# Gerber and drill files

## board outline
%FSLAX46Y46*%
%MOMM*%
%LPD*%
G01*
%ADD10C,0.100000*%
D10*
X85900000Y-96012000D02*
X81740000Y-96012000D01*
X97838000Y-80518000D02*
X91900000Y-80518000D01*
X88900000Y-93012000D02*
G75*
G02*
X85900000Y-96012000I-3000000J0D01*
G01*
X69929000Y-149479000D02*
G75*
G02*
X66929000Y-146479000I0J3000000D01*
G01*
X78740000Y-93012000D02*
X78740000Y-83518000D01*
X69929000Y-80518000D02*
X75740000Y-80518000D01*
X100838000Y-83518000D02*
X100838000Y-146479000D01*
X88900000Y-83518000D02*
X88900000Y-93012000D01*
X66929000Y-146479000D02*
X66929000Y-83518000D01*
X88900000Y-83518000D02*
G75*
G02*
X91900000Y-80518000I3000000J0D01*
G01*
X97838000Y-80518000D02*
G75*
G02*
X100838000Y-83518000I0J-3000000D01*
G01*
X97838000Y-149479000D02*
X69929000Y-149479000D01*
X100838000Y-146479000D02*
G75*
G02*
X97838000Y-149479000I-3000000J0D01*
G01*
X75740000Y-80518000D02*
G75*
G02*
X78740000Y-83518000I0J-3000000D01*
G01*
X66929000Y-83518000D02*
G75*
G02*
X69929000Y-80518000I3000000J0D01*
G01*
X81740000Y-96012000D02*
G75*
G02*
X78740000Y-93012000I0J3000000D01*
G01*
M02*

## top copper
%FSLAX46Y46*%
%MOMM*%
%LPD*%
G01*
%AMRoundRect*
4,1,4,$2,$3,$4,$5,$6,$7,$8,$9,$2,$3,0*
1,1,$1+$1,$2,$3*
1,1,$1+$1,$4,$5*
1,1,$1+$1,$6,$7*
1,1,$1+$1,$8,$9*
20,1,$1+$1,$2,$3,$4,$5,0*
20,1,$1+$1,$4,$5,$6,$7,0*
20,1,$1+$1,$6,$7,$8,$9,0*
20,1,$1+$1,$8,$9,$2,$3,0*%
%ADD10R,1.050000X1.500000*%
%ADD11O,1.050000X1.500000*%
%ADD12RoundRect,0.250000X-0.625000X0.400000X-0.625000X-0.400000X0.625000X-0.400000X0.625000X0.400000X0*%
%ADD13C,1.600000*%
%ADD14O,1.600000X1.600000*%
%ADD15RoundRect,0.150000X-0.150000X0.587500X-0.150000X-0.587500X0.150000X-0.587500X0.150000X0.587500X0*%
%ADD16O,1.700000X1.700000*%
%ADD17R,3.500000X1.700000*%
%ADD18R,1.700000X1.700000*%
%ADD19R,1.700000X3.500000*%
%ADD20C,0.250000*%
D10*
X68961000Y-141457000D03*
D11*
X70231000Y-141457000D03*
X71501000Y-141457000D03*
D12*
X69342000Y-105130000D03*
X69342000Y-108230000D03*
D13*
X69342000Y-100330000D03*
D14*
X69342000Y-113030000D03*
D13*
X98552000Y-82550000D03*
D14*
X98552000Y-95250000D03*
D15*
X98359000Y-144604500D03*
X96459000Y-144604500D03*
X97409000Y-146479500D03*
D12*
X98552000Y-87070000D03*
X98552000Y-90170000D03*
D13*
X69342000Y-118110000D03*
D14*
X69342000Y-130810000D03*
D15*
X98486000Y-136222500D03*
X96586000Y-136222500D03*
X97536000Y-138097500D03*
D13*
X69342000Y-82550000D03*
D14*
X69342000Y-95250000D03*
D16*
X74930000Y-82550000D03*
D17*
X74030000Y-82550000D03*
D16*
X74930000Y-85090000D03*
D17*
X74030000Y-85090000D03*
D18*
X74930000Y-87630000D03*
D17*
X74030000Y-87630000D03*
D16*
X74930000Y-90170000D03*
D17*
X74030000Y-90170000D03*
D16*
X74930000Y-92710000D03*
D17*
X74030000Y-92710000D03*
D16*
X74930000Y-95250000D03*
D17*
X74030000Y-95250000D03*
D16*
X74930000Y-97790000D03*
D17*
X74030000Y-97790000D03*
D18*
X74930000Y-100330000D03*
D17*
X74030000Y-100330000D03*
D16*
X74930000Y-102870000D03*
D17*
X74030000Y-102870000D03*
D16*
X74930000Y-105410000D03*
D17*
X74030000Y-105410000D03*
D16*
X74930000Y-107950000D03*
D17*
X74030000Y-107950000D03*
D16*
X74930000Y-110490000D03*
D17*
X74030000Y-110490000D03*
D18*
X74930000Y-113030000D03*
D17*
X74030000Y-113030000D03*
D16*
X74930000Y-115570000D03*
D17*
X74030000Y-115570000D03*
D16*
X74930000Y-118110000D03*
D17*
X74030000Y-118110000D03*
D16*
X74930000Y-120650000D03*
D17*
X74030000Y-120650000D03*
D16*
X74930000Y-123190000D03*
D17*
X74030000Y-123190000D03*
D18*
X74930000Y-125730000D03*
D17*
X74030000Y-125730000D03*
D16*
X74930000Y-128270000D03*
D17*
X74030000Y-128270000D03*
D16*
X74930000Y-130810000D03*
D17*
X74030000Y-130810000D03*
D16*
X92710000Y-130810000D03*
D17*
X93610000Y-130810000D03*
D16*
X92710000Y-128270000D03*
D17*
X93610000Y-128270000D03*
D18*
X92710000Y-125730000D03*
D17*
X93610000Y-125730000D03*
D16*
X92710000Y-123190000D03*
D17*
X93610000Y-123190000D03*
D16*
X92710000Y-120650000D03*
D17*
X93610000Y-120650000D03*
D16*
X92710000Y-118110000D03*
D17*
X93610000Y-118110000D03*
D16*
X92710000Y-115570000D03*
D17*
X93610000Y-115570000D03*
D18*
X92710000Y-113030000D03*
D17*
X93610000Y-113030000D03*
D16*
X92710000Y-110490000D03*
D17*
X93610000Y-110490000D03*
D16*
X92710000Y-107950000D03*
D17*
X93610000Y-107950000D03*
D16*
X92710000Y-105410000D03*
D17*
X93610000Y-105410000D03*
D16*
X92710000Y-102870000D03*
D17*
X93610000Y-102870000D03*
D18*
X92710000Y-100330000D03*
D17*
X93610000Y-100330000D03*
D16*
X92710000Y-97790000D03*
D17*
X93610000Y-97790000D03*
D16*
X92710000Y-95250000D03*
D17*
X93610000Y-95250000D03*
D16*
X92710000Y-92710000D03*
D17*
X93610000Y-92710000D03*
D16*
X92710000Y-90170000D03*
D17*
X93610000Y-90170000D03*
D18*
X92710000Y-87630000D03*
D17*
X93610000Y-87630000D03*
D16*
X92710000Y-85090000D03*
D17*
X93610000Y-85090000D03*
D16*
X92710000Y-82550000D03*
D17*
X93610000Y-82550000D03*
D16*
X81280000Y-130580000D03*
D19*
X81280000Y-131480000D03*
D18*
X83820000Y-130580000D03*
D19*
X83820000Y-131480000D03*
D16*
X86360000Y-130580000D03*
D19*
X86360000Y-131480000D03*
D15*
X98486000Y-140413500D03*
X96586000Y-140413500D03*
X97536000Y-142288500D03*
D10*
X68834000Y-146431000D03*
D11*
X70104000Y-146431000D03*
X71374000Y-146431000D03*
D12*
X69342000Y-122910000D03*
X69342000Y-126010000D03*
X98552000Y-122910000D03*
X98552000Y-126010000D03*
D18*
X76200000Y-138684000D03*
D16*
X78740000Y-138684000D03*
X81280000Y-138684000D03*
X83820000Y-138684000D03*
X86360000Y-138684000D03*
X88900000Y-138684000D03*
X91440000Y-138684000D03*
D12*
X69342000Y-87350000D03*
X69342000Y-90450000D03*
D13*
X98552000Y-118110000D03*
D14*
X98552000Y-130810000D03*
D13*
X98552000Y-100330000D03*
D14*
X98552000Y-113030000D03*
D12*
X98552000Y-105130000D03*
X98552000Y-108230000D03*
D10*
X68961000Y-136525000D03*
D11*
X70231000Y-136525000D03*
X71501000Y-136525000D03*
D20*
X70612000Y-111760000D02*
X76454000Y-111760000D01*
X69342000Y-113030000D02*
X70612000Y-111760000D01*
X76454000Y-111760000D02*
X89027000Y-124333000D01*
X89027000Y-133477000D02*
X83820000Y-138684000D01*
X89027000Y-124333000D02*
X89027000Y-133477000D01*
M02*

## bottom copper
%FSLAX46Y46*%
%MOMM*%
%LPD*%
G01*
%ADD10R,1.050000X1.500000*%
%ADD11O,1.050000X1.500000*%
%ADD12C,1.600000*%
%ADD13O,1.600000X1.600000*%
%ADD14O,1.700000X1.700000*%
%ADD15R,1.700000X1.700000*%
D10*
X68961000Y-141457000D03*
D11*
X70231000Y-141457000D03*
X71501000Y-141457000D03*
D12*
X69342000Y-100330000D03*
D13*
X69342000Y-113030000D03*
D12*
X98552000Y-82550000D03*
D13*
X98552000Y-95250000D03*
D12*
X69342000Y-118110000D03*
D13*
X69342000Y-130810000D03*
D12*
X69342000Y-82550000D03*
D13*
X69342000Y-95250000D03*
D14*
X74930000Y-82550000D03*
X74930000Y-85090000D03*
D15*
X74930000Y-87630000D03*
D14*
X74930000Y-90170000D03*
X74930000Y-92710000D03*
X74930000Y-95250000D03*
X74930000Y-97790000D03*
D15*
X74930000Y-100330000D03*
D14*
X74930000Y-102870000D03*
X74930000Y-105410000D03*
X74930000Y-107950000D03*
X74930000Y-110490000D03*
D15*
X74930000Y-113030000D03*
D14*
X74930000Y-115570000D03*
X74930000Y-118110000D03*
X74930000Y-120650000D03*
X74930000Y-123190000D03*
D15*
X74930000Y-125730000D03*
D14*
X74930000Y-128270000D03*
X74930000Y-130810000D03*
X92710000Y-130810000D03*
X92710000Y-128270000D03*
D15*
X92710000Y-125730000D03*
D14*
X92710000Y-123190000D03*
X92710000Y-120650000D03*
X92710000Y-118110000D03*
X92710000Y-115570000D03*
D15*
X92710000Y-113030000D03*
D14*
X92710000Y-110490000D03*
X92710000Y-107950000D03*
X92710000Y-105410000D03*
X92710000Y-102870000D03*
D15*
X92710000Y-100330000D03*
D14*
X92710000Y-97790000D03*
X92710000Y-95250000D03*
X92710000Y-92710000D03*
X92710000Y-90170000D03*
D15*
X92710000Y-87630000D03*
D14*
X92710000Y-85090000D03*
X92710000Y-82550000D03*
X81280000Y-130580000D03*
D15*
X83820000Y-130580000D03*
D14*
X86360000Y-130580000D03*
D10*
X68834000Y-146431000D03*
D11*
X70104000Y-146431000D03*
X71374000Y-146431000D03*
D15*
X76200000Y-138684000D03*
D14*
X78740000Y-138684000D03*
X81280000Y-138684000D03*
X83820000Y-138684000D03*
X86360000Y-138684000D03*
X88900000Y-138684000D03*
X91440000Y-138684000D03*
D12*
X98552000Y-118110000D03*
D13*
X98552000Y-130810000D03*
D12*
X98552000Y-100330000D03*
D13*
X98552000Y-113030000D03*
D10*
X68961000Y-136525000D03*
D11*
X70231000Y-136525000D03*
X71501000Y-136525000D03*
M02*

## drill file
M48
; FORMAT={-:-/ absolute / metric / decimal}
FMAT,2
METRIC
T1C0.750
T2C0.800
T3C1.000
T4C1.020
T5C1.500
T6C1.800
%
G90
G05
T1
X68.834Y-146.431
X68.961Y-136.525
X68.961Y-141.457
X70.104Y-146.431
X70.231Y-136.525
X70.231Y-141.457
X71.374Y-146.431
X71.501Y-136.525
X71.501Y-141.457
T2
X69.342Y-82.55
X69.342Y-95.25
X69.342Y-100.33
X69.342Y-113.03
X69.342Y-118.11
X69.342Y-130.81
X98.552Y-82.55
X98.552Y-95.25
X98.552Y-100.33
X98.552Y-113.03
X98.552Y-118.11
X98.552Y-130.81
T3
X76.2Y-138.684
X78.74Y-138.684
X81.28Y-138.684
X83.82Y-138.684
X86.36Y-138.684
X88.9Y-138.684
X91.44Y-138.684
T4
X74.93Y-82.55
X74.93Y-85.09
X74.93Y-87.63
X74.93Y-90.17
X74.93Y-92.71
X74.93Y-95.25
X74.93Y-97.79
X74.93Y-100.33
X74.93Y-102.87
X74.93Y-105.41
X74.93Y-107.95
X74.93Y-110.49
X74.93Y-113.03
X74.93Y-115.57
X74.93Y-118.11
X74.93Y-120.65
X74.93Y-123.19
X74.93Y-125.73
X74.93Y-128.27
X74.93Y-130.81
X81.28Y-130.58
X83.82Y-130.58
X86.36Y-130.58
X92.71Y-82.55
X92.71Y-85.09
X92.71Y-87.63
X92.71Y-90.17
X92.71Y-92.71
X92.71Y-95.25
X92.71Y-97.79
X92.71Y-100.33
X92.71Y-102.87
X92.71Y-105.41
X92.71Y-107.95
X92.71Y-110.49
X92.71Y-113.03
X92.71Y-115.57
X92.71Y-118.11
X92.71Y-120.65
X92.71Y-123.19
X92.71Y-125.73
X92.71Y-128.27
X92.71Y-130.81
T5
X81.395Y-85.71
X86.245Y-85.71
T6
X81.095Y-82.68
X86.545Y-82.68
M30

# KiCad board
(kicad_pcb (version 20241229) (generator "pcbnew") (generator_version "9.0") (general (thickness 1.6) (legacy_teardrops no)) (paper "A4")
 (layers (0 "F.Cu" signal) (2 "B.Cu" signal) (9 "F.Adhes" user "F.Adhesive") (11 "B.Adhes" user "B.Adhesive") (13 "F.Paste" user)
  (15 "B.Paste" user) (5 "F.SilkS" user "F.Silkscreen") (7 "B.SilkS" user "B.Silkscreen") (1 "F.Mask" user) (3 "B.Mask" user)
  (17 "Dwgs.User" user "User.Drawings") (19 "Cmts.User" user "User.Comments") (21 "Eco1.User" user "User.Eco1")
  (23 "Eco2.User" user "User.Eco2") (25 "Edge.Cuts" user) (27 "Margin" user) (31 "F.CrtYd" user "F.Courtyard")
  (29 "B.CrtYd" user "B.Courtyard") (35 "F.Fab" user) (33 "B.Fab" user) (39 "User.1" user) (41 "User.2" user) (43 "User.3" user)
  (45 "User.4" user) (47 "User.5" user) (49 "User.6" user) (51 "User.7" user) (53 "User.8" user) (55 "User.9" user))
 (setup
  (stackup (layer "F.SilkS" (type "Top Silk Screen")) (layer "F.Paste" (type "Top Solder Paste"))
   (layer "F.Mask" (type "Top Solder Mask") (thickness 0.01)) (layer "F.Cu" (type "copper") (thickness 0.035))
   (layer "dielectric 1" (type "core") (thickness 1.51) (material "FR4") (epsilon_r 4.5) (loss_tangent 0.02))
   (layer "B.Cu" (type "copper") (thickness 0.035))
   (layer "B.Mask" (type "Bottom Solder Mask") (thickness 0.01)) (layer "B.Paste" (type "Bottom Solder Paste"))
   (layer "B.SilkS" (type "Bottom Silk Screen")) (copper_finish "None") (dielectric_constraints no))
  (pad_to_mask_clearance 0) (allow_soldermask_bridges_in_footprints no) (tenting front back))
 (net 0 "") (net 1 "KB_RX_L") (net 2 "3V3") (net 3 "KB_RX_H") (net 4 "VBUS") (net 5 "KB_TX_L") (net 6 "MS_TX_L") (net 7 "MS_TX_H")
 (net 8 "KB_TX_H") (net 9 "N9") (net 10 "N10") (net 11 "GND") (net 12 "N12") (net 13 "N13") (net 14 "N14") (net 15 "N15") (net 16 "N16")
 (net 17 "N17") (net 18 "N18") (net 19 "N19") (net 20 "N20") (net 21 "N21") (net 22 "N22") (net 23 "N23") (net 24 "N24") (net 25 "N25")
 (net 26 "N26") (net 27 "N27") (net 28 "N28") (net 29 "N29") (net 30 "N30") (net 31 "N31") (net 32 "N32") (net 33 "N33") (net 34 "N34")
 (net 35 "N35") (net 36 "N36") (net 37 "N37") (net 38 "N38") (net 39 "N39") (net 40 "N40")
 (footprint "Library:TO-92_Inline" (layer "F.Cu") (at 68.961 141.457)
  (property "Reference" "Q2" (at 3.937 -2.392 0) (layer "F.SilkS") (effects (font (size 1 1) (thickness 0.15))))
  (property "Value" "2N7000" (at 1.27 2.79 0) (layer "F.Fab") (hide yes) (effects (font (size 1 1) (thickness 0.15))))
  (pad "1" thru_hole rect (at 0 0) (size 1.05 1.5) (drill 0.75) (layers "*.Cu" "*.Mask") (remove_unused_layers no) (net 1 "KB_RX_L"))
  (pad "2" thru_hole oval (at 1.27 0) (size 1.05 1.5) (drill 0.75) (layers "*.Cu" "*.Mask") (remove_unused_layers no) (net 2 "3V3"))
  (pad "3" thru_hole oval (at 2.54 0) (size 1.05 1.5) (drill 0.75) (layers "*.Cu" "*.Mask") (remove_unused_layers no) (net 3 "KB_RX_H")))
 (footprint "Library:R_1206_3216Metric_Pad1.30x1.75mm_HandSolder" (layer "F.Cu") (at 69.342 106.68 -90)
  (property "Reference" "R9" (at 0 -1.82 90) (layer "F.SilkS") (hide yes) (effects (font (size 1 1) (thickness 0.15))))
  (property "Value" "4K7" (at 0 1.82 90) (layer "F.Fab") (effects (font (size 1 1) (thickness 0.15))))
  (pad "1" smd roundrect (at -1.55 0 270) (size 1.3 1.75) (layers "F.Cu" "F.Mask" "F.Paste") (roundrect_rratio 0.192308) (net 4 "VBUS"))
  (pad "2" smd roundrect (at 1.55 0 270) (size 1.3 1.75) (layers "F.Cu" "F.Mask" "F.Paste") (roundrect_rratio 0.192308) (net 3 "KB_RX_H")))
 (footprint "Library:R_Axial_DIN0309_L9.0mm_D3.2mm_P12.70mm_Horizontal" (layer "F.Cu") (at 69.342 100.33 -90)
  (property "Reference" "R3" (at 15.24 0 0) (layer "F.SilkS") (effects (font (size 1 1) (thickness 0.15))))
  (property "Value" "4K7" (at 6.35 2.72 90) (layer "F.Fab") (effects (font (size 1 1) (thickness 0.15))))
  (pad "1" thru_hole circle (at 0 0 270) (size 1.6 1.6) (drill 0.8) (layers "*.Cu" "*.Mask") (remove_unused_layers no) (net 4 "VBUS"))
  (pad "2" thru_hole oval (at 12.7 0 270) (size 1.6 1.6) (drill 0.8) (layers "*.Cu" "*.Mask") (remove_unused_layers no) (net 3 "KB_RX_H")))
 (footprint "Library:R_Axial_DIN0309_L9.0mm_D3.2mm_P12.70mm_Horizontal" (layer "F.Cu") (at 98.552 82.55 -90)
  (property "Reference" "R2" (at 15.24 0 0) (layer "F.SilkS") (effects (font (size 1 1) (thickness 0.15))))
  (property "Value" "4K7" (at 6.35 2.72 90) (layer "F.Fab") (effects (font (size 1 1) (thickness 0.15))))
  (pad "1" thru_hole circle (at 0 0 270) (size 1.6 1.6) (drill 0.8) (layers "*.Cu" "*.Mask") (remove_unused_layers no) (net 2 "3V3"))
  (pad "2" thru_hole oval (at 12.7 0 270) (size 1.6 1.6) (drill 0.8) (layers "*.Cu" "*.Mask") (remove_unused_layers no) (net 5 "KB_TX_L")))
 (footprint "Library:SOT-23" (layer "F.Cu") (at 97.409 145.542 -90)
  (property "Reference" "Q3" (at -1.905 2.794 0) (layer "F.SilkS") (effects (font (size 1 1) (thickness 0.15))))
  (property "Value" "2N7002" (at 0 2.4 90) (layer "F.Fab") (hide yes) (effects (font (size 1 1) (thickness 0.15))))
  (pad "1" smd roundrect (at -0.9375 -0.95 270) (size 1.475 0.6) (layers "F.Cu" "F.Mask" "F.Paste") (roundrect_rratio 0.25) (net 2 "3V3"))
  (pad "2" smd roundrect (at -0.9375 0.95 270) (size 1.475 0.6) (layers "F.Cu" "F.Mask" "F.Paste") (roundrect_rratio 0.25) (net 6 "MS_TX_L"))
  (pad "3" smd roundrect (at 0.9375 0 270) (size 1.475 0.6) (layers "F.Cu" "F.Mask" "F.Paste") (roundrect_rratio 0.25) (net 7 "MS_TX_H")))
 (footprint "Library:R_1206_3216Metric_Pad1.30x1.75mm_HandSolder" (layer "F.Cu") (at 98.552 88.62 -90)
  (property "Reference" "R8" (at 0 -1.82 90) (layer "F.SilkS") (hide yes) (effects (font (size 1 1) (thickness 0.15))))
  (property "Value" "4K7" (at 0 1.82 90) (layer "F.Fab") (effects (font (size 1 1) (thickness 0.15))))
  (pad "1" smd roundrect (at -1.55 0 270) (size 1.3 1.75) (layers "F.Cu" "F.Mask" "F.Paste") (roundrect_rratio 0.192308) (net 2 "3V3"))
  (pad "2" smd roundrect (at 1.55 0 270) (size 1.3 1.75) (layers "F.Cu" "F.Mask" "F.Paste") (roundrect_rratio 0.192308) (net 5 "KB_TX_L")))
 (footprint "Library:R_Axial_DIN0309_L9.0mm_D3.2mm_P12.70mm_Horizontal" (layer "F.Cu") (at 69.342 118.11 -90)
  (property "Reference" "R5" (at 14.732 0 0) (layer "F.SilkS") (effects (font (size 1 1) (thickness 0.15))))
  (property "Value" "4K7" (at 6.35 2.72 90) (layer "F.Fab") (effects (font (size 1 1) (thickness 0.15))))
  (pad "1" thru_hole circle (at 0 0 270) (size 1.6 1.6) (drill 0.8) (layers "*.Cu" "*.Mask") (remove_unused_layers no) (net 4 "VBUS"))
  (pad "2" thru_hole oval (at 12.7 0 270) (size 1.6 1.6) (drill 0.8) (layers "*.Cu" "*.Mask") (remove_unused_layers no) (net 7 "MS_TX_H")))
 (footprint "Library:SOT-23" (layer "F.Cu") (at 97.536 137.16 -90)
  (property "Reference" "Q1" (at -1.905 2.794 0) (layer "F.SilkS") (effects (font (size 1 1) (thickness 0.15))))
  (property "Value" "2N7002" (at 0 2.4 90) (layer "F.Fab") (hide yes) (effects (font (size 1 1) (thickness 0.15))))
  (pad "1" smd roundrect (at -0.9375 -0.95 270) (size 1.475 0.6) (layers "F.Cu" "F.Mask" "F.Paste") (roundrect_rratio 0.25) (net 2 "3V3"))
  (pad "2" smd roundrect (at -0.9375 0.95 270) (size 1.475 0.6) (layers "F.Cu" "F.Mask" "F.Paste") (roundrect_rratio 0.25) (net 5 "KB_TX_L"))
  (pad "3" smd roundrect (at 0.9375 0 270) (size 1.475 0.6) (layers "F.Cu" "F.Mask" "F.Paste") (roundrect_rratio 0.25) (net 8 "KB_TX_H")))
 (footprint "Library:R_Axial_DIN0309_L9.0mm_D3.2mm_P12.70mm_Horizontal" (layer "F.Cu") (at 69.342 82.55 -90)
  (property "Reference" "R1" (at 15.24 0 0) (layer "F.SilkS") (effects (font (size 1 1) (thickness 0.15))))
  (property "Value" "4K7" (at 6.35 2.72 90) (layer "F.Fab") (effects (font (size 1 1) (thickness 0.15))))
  (pad "1" thru_hole circle (at 0 0 270) (size 1.6 1.6) (drill 0.8) (layers "*.Cu" "*.Mask") (remove_unused_layers no) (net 4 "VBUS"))
  (pad "2" thru_hole oval (at 12.7 0 270) (size 1.6 1.6) (drill 0.8) (layers "*.Cu" "*.Mask") (remove_unused_layers no) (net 8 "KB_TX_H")))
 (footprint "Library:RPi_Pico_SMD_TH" (layer "F.Cu") (at 83.82 106.68)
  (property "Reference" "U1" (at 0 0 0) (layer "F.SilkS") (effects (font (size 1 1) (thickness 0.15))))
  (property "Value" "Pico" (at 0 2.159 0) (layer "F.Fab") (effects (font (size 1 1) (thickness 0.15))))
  (pad "" np_thru_hole oval (at -2.725 -24) (size 1.8 1.8) (drill 1.8) (layers "*.Cu" "*.Mask"))
  (pad "" np_thru_hole oval (at -2.425 -20.97) (size 1.5 1.5) (drill 1.5) (layers "*.Cu" "*.Mask"))
  (pad "" np_thru_hole oval (at 2.425 -20.97) (size 1.5 1.5) (drill 1.5) (layers "*.Cu" "*.Mask"))
  (pad "" np_thru_hole oval (at 2.725 -24) (size 1.8 1.8) (drill 1.8) (layers "*.Cu" "*.Mask"))
  (pad "1" thru_hole oval (at -8.89 -24.13) (size 1.7 1.7) (drill 1.02) (layers "*.Cu" "*.Mask") (remove_unused_layers no) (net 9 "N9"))
  (pad "1" smd rect (at -8.89 -24.13) (size 3.5 1.7) (drill (offset -0.9 0)) (layers "F.Cu" "F.Mask") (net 9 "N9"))
  (pad "2" thru_hole oval (at -8.89 -21.59) (size 1.7 1.7) (drill 1.02) (layers "*.Cu" "*.Mask") (remove_unused_layers no) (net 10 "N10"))
  (pad "2" smd rect (at -8.89 -21.59) (size 3.5 1.7) (drill (offset -0.9 0)) (layers "F.Cu" "F.Mask") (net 10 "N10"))
  (pad "3" thru_hole rect (at -8.89 -19.05) (size 1.7 1.7) (drill 1.02) (layers "*.Cu" "*.Mask") (remove_unused_layers no) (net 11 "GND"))
  (pad "3" smd rect (at -8.89 -19.05) (size 3.5 1.7) (drill (offset -0.9 0)) (layers "F.Cu" "F.Mask") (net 11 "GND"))
  (pad "4" thru_hole oval (at -8.89 -16.51) (size 1.7 1.7) (drill 1.02) (layers "*.Cu" "*.Mask") (remove_unused_layers no) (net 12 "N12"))
  (pad "4" smd rect (at -8.89 -16.51) (size 3.5 1.7) (drill (offset -0.9 0)) (layers "F.Cu" "F.Mask") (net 12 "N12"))
  (pad "5" thru_hole oval (at -8.89 -13.97) (size 1.7 1.7) (drill 1.02) (layers "*.Cu" "*.Mask") (remove_unused_layers no) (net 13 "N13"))
  (pad "5" smd rect (at -8.89 -13.97) (size 3.5 1.7) (drill (offset -0.9 0)) (layers "F.Cu" "F.Mask") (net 13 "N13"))
  (pad "6" thru_hole oval (at -8.89 -11.43) (size 1.7 1.7) (drill 1.02) (layers "*.Cu" "*.Mask") (remove_unused_layers no) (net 5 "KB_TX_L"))
  (pad "6" smd rect (at -8.89 -11.43) (size 3.5 1.7) (drill (offset -0.9 0)) (layers "F.Cu" "F.Mask") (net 5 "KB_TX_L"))
  (pad "7" thru_hole oval (at -8.89 -8.89) (size 1.7 1.7) (drill 1.02) (layers "*.Cu" "*.Mask") (remove_unused_layers no) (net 1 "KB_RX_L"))
  (pad "7" smd rect (at -8.89 -8.89) (size 3.5 1.7) (drill (offset -0.9 0)) (layers "F.Cu" "F.Mask") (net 1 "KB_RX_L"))
  (pad "8" thru_hole rect (at -8.89 -6.35) (size 1.7 1.7) (drill 1.02) (layers "*.Cu" "*.Mask") (remove_unused_layers no) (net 11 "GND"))
  (pad "8" smd rect (at -8.89 -6.35) (size 3.5 1.7) (drill (offset -0.9 0)) (layers "F.Cu" "F.Mask") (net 11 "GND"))
  (pad "9" thru_hole oval (at -8.89 -3.81) (size 1.7 1.7) (drill 1.02) (layers "*.Cu" "*.Mask") (remove_unused_layers no) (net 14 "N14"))
  (pad "9" smd rect (at -8.89 -3.81) (size 3.5 1.7) (drill (offset -0.9 0)) (layers "F.Cu" "F.Mask") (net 14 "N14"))
  (pad "10" thru_hole oval (at -8.89 -1.27) (size 1.7 1.7) (drill 1.02) (layers "*.Cu" "*.Mask") (remove_unused_layers no) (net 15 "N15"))
  (pad "10" smd rect (at -8.89 -1.27) (size 3.5 1.7) (drill (offset -0.9 0)) (layers "F.Cu" "F.Mask") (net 15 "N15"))
  (pad "11" thru_hole oval (at -8.89 1.27) (size 1.7 1.7) (drill 1.02) (layers "*.Cu" "*.Mask") (remove_unused_layers no) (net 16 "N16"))
  (pad "11" smd rect (at -8.89 1.27) (size 3.5 1.7) (drill (offset -0.9 0)) (layers "F.Cu" "F.Mask") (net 16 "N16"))
  (pad "12" thru_hole oval (at -8.89 3.81) (size 1.7 1.7) (drill 1.02) (layers "*.Cu" "*.Mask") (remove_unused_layers no) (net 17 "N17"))
  (pad "12" smd rect (at -8.89 3.81) (size 3.5 1.7) (drill (offset -0.9 0)) (layers "F.Cu" "F.Mask") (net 17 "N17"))
  (pad "13" thru_hole rect (at -8.89 6.35) (size 1.7 1.7) (drill 1.02) (layers "*.Cu" "*.Mask") (remove_unused_layers no) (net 11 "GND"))
  (pad "13" smd rect (at -8.89 6.35) (size 3.5 1.7) (drill (offset -0.9 0)) (layers "F.Cu" "F.Mask") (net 11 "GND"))
  (pad "14" thru_hole oval (at -8.89 8.89) (size 1.7 1.7) (drill 1.02) (layers "*.Cu" "*.Mask") (remove_unused_layers no) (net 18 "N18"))
  (pad "14" smd rect (at -8.89 8.89) (size 3.5 1.7) (drill (offset -0.9 0)) (layers "F.Cu" "F.Mask") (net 18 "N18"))
  (pad "15" thru_hole oval (at -8.89 11.43) (size 1.7 1.7) (drill 1.02) (layers "*.Cu" "*.Mask") (remove_unused_layers no) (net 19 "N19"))
  (pad "15" smd rect (at -8.89 11.43) (size 3.5 1.7) (drill (offset -0.9 0)) (layers "F.Cu" "F.Mask") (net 19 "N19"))
  (pad "16" thru_hole oval (at -8.89 13.97) (size 1.7 1.7) (drill 1.02) (layers "*.Cu" "*.Mask") (remove_unused_layers no) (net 6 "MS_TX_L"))
  (pad "16" smd rect (at -8.89 13.97) (size 3.5 1.7) (drill (offset -0.9 0)) (layers "F.Cu" "F.Mask") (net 6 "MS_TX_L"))
  (pad "17" thru_hole oval (at -8.89 16.51) (size 1.7 1.7) (drill 1.02) (layers "*.Cu" "*.Mask") (remove_unused_layers no) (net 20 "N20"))
  (pad "17" smd rect (at -8.89 16.51) (size 3.5 1.7) (drill (offset -0.9 0)) (layers "F.Cu" "F.Mask") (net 20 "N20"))
  (pad "18" thru_hole rect (at -8.89 19.05) (size 1.7 1.7) (drill 1.02) (layers "*.Cu" "*.Mask") (remove_unused_layers no) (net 11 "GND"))
  (pad "18" smd rect (at -8.89 19.05) (size 3.5 1.7) (drill (offset -0.9 0)) (layers "F.Cu" "F.Mask") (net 11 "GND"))
  (pad "19" thru_hole oval (at -8.89 21.59) (size 1.7 1.7) (drill 1.02) (layers "*.Cu" "*.Mask") (remove_unused_layers no) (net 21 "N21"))
  (pad "19" smd rect (at -8.89 21.59) (size 3.5 1.7) (drill (offset -0.9 0)) (layers "F.Cu" "F.Mask") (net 21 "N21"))
  (pad "20" thru_hole oval (at -8.89 24.13) (size 1.7 1.7) (drill 1.02) (layers "*.Cu" "*.Mask") (remove_unused_layers no) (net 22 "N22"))
  (pad "20" smd rect (at -8.89 24.13) (size 3.5 1.7) (drill (offset -0.9 0)) (layers "F.Cu" "F.Mask") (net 22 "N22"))
  (pad "21" thru_hole oval (at 8.89 24.13) (size 1.7 1.7) (drill 1.02) (layers "*.Cu" "*.Mask") (remove_unused_layers no) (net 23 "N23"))
  (pad "21" smd rect (at 8.89 24.13) (size 3.5 1.7) (drill (offset 0.9 0)) (layers "F.Cu" "F.Mask") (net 23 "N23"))
  (pad "22" thru_hole oval (at 8.89 21.59) (size 1.7 1.7) (drill 1.02) (layers "*.Cu" "*.Mask") (remove_unused_layers no) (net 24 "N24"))
  (pad "22" smd rect (at 8.89 21.59) (size 3.5 1.7) (drill (offset 0.9 0)) (layers "F.Cu" "F.Mask") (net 24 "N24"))
  (pad "23" thru_hole rect (at 8.89 19.05) (size 1.7 1.7) (drill 1.02) (layers "*.Cu" "*.Mask") (remove_unused_layers no) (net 11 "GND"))
  (pad "23" smd rect (at 8.89 19.05) (size 3.5 1.7) (drill (offset 0.9 0)) (layers "F.Cu" "F.Mask") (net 11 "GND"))
  (pad "24" thru_hole oval (at 8.89 16.51) (size 1.7 1.7) (drill 1.02) (layers "*.Cu" "*.Mask") (remove_unused_layers no) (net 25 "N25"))
  (pad "24" smd rect (at 8.89 16.51) (size 3.5 1.7) (drill (offset 0.9 0)) (layers "F.Cu" "F.Mask") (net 25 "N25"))
  (pad "25" thru_hole oval (at 8.89 13.97) (size 1.7 1.7) (drill 1.02) (layers "*.Cu" "*.Mask") (remove_unused_layers no) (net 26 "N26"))
  (pad "25" smd rect (at 8.89 13.97) (size 3.5 1.7) (drill (offset 0.9 0)) (layers "F.Cu" "F.Mask") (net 26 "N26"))
  (pad "26" thru_hole oval (at 8.89 11.43) (size 1.7 1.7) (drill 1.02) (layers "*.Cu" "*.Mask") (remove_unused_layers no) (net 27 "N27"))
  (pad "26" smd rect (at 8.89 11.43) (size 3.5 1.7) (drill (offset 0.9 0)) (layers "F.Cu" "F.Mask") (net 27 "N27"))
  (pad "27" thru_hole oval (at 8.89 8.89) (size 1.7 1.7) (drill 1.02) (layers "*.Cu" "*.Mask") (remove_unused_layers no) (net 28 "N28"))
  (pad "27" smd rect (at 8.89 8.89) (size 3.5 1.7) (drill (offset 0.9 0)) (layers "F.Cu" "F.Mask") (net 28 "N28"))
  (pad "28" thru_hole rect (at 8.89 6.35) (size 1.7 1.7) (drill 1.02) (layers "*.Cu" "*.Mask") (remove_unused_layers no) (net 11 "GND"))
  (pad "28" smd rect (at 8.89 6.35) (size 3.5 1.7) (drill (offset 0.9 0)) (layers "F.Cu" "F.Mask") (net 11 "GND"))
  (pad "29" thru_hole oval (at 8.89 3.81) (size 1.7 1.7) (drill 1.02) (layers "*.Cu" "*.Mask") (remove_unused_layers no) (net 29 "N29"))
  (pad "29" smd rect (at 8.89 3.81) (size 3.5 1.7) (drill (offset 0.9 0)) (layers "F.Cu" "F.Mask") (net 29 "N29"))
  (pad "30" thru_hole oval (at 8.89 1.27) (size 1.7 1.7) (drill 1.02) (layers "*.Cu" "*.Mask") (remove_unused_layers no) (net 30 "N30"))
  (pad "30" smd rect (at 8.89 1.27) (size 3.5 1.7) (drill (offset 0.9 0)) (layers "F.Cu" "F.Mask") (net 30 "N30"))
  (pad "31" thru_hole oval (at 8.89 -1.27) (size 1.7 1.7) (drill 1.02) (layers "*.Cu" "*.Mask") (remove_unused_layers no) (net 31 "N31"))
  (pad "31" smd rect (at 8.89 -1.27) (size 3.5 1.7) (drill (offset 0.9 0)) (layers "F.Cu" "F.Mask") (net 31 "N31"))
  (pad "32" thru_hole oval (at 8.89 -3.81) (size 1.7 1.7) (drill 1.02) (layers "*.Cu" "*.Mask") (remove_unused_layers no) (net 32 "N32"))
  (pad "32" smd rect (at 8.89 -3.81) (size 3.5 1.7) (drill (offset 0.9 0)) (layers "F.Cu" "F.Mask") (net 32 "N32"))
  (pad "33" thru_hole rect (at 8.89 -6.35) (size 1.7 1.7) (drill 1.02) (layers "*.Cu" "*.Mask") (remove_unused_layers no) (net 11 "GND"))
  (pad "33" smd rect (at 8.89 -6.35) (size 3.5 1.7) (drill (offset 0.9 0)) (layers "F.Cu" "F.Mask") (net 11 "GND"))
  (pad "34" thru_hole oval (at 8.89 -8.89) (size 1.7 1.7) (drill 1.02) (layers "*.Cu" "*.Mask") (remove_unused_layers no) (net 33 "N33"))
  (pad "34" smd rect (at 8.89 -8.89) (size 3.5 1.7) (drill (offset 0.9 0)) (layers "F.Cu" "F.Mask") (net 33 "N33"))
  (pad "35" thru_hole oval (at 8.89 -11.43) (size 1.7 1.7) (drill 1.02) (layers "*.Cu" "*.Mask") (remove_unused_layers no) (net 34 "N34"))
  (pad "35" smd rect (at 8.89 -11.43) (size 3.5 1.7) (drill (offset 0.9 0)) (layers "F.Cu" "F.Mask") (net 34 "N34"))
  (pad "36" thru_hole oval (at 8.89 -13.97) (size 1.7 1.7) (drill 1.02) (layers "*.Cu" "*.Mask") (remove_unused_layers no) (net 2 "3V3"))
  (pad "36" smd rect (at 8.89 -13.97) (size 3.5 1.7) (drill (offset 0.9 0)) (layers "F.Cu" "F.Mask") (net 2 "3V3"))
  (pad "37" thru_hole oval (at 8.89 -16.51) (size 1.7 1.7) (drill 1.02) (layers "*.Cu" "*.Mask") (remove_unused_layers no) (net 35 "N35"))
  (pad "37" smd rect (at 8.89 -16.51) (size 3.5 1.7) (drill (offset 0.9 0)) (layers "F.Cu" "F.Mask") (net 35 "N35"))
  (pad "38" thru_hole rect (at 8.89 -19.05) (size 1.7 1.7) (drill 1.02) (layers "*.Cu" "*.Mask") (remove_unused_layers no) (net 11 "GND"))
  (pad "38" smd rect (at 8.89 -19.05) (size 3.5 1.7) (drill (offset 0.9 0)) (layers "F.Cu" "F.Mask") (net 11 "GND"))
  (pad "39" thru_hole oval (at 8.89 -21.59) (size 1.7 1.7) (drill 1.02) (layers "*.Cu" "*.Mask") (remove_unused_layers no) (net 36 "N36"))
  (pad "39" smd rect (at 8.89 -21.59) (size 3.5 1.7) (drill (offset 0.9 0)) (layers "F.Cu" "F.Mask") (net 36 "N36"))
  (pad "40" thru_hole oval (at 8.89 -24.13) (size 1.7 1.7) (drill 1.02) (layers "*.Cu" "*.Mask") (remove_unused_layers no) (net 4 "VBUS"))
  (pad "40" smd rect (at 8.89 -24.13) (size 3.5 1.7) (drill (offset 0.9 0)) (layers "F.Cu" "F.Mask") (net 4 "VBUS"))
  (pad "41" thru_hole oval (at -2.54 23.9) (size 1.7 1.7) (drill 1.02) (layers "*.Cu" "*.Mask") (remove_unused_layers no) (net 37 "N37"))
  (pad "41" smd rect (at -2.54 23.9 90) (size 3.5 1.7) (drill (offset -0.9 0)) (layers "F.Cu" "F.Mask") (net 37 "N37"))
  (pad "42" thru_hole rect (at 0 23.9) (size 1.7 1.7) (drill 1.02) (layers "*.Cu" "*.Mask") (remove_unused_layers no) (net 11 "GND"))
  (pad "42" smd rect (at 0 23.9 90) (size 3.5 1.7) (drill (offset -0.9 0)) (layers "F.Cu" "F.Mask") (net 11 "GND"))
  (pad "43" thru_hole oval (at 2.54 23.9) (size 1.7 1.7) (drill 1.02) (layers "*.Cu" "*.Mask") (remove_unused_layers no) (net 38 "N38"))
  (pad "43" smd rect (at 2.54 23.9 90) (size 3.5 1.7) (drill (offset -0.9 0)) (layers "F.Cu" "F.Mask") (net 38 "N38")))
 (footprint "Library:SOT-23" (layer "F.Cu") (at 97.536 141.351 -90)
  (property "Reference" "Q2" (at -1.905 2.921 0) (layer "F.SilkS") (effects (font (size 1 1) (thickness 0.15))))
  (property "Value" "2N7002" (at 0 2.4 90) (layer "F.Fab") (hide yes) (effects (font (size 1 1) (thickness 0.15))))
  (pad "1" smd roundrect (at -0.9375 -0.95 270) (size 1.475 0.6) (layers "F.Cu" "F.Mask" "F.Paste") (roundrect_rratio 0.25) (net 2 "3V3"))
  (pad "2" smd roundrect (at -0.9375 0.95 270) (size 1.475 0.6) (layers "F.Cu" "F.Mask" "F.Paste") (roundrect_rratio 0.25) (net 1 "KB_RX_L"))
  (pad "3" smd roundrect (at 0.9375 0 270) (size 1.475 0.6) (layers "F.Cu" "F.Mask" "F.Paste") (roundrect_rratio 0.25) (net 3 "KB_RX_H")))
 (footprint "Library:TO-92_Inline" (layer "F.Cu") (at 68.834 146.431)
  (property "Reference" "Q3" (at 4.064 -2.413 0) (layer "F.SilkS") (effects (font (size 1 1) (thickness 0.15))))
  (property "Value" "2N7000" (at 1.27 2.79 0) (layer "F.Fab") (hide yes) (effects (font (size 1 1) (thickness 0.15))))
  (pad "1" thru_hole rect (at 0 0) (size 1.05 1.5) (drill 0.75) (layers "*.Cu" "*.Mask") (remove_unused_layers no) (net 6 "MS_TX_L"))
  (pad "2" thru_hole oval (at 1.27 0) (size 1.05 1.5) (drill 0.75) (layers "*.Cu" "*.Mask") (remove_unused_layers no) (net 2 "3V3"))
  (pad "3" thru_hole oval (at 2.54 0) (size 1.05 1.5) (drill 0.75) (layers "*.Cu" "*.Mask") (remove_unused_layers no) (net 7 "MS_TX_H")))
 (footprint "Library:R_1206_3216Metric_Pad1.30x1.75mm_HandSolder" (layer "F.Cu") (at 69.342 124.46 -90)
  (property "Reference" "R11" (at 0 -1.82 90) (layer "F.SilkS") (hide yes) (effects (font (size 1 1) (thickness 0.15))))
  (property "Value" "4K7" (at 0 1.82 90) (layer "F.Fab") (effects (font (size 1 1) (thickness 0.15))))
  (pad "1" smd roundrect (at -1.55 0 270) (size 1.3 1.75) (layers "F.Cu" "F.Mask" "F.Paste") (roundrect_rratio 0.192308) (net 4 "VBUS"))
  (pad "2" smd roundrect (at 1.55 0 270) (size 1.3 1.75) (layers "F.Cu" "F.Mask" "F.Paste") (roundrect_rratio 0.192308) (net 7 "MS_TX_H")))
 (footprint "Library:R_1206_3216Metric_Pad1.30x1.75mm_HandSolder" (layer "F.Cu") (at 98.552 124.46 -90)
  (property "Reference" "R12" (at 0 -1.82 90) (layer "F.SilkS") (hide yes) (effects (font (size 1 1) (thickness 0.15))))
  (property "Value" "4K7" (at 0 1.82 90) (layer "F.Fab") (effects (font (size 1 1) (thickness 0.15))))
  (pad "1" smd roundrect (at -1.55 0 270) (size 1.3 1.75) (layers "F.Cu" "F.Mask" "F.Paste") (roundrect_rratio 0.192308) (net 2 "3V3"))
  (pad "2" smd roundrect (at 1.55 0 270) (size 1.3 1.75) (layers "F.Cu" "F.Mask" "F.Paste") (roundrect_rratio 0.192308) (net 6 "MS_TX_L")))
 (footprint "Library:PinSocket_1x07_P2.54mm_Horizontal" (layer "F.Cu") (at 76.2 138.684 90)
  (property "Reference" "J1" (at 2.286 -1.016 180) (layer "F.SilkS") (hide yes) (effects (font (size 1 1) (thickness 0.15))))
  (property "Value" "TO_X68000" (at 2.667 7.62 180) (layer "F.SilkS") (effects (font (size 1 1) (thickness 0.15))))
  (pad "1" thru_hole rect (at 0 0 90) (size 1.7 1.7) (drill 1) (layers "*.Cu" "*.Mask") (remove_unused_layers no) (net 4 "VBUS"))
  (pad "2" thru_hole oval (at 0 2.54 90) (size 1.7 1.7) (drill 1) (layers "*.Cu" "*.Mask") (remove_unused_layers no) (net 7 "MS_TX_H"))
  (pad "3" thru_hole oval (at 0 5.08 90) (size 1.7 1.7) (drill 1) (layers "*.Cu" "*.Mask") (remove_unused_layers no) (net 8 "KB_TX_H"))
  (pad "4" thru_hole oval (at 0 7.62 90) (size 1.7 1.7) (drill 1) (layers "*.Cu" "*.Mask") (remove_unused_layers no) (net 3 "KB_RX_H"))
  (pad "5" thru_hole oval (at 0 10.16 90) (size 1.7 1.7) (drill 1) (layers "*.Cu" "*.Mask") (remove_unused_layers no) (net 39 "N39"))
  (pad "6" thru_hole oval (at 0 12.7 90) (size 1.7 1.7) (drill 1) (layers "*.Cu" "*.Mask") (remove_unused_layers no) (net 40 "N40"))
  (pad "7" thru_hole oval (at 0 15.24 90) (size 1.7 1.7) (drill 1) (layers "*.Cu" "*.Mask") (remove_unused_layers no) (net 11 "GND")))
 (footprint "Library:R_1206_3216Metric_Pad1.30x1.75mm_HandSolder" (layer "F.Cu") (at 69.342 88.9 -90)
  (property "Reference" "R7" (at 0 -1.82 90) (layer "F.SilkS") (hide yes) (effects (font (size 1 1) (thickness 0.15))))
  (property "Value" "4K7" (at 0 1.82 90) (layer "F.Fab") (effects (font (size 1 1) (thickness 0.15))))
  (pad "1" smd roundrect (at -1.55 0 270) (size 1.3 1.75) (layers "F.Cu" "F.Mask" "F.Paste") (roundrect_rratio 0.192308) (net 4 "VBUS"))
  (pad "2" smd roundrect (at 1.55 0 270) (size 1.3 1.75) (layers "F.Cu" "F.Mask" "F.Paste") (roundrect_rratio 0.192308) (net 8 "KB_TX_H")))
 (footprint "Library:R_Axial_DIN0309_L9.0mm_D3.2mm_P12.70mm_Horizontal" (layer "F.Cu") (at 98.552 118.11 -90)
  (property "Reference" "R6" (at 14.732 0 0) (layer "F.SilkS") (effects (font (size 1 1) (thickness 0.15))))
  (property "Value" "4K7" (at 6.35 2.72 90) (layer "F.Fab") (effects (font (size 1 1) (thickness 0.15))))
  (pad "1" thru_hole circle (at 0 0 270) (size 1.6 1.6) (drill 0.8) (layers "*.Cu" "*.Mask") (remove_unused_layers no) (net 2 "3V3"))
  (pad "2" thru_hole oval (at 12.7 0 270) (size 1.6 1.6) (drill 0.8) (layers "*.Cu" "*.Mask") (remove_unused_layers no) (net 6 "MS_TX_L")))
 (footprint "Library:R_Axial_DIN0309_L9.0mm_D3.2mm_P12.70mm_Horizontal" (layer "F.Cu") (at 98.552 100.33 -90)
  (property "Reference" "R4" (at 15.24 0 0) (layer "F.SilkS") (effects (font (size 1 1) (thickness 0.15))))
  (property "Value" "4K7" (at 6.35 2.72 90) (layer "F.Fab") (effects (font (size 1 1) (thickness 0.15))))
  (pad "1" thru_hole circle (at 0 0 270) (size 1.6 1.6) (drill 0.8) (layers "*.Cu" "*.Mask") (remove_unused_layers no) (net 2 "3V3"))
  (pad "2" thru_hole oval (at 12.7 0 270) (size 1.6 1.6) (drill 0.8) (layers "*.Cu" "*.Mask") (remove_unused_layers no) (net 1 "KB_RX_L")))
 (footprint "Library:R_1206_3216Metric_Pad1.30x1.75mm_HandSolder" (layer "F.Cu") (at 98.552 106.68 -90)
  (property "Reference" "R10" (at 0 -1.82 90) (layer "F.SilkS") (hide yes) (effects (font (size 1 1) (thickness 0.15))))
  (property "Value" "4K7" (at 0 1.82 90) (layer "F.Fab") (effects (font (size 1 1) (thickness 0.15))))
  (pad "1" smd roundrect (at -1.55 0 270) (size 1.3 1.75) (layers "F.Cu" "F.Mask" "F.Paste") (roundrect_rratio 0.192308) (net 2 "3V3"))
  (pad "2" smd roundrect (at 1.55 0 270) (size 1.3 1.75) (layers "F.Cu" "F.Mask" "F.Paste") (roundrect_rratio 0.192308) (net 1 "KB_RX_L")))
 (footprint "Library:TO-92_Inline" (layer "F.Cu") (at 68.961 136.525)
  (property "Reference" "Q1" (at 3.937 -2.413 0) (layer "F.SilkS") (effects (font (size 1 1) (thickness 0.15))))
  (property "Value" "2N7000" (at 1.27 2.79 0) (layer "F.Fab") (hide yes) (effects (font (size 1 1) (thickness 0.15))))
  (pad "1" thru_hole rect (at 0 0) (size 1.05 1.5) (drill 0.75) (layers "*.Cu" "*.Mask") (remove_unused_layers no) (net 5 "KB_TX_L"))
  (pad "2" thru_hole oval (at 1.27 0) (size 1.05 1.5) (drill 0.75) (layers "*.Cu" "*.Mask") (remove_unused_layers no) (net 2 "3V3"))
  (pad "3" thru_hole oval (at 2.54 0) (size 1.05 1.5) (drill 0.75) (layers "*.Cu" "*.Mask") (remove_unused_layers no) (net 8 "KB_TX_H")))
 (gr_line (start 85.9 96.012) (end 81.74 96.012) (stroke (width 0.1) (type default)) (layer "Edge.Cuts"))
 (gr_line (start 97.838 80.518) (end 91.9 80.518) (stroke (width 0.1) (type default)) (layer "Edge.Cuts"))
 (gr_arc (start 88.9 93.012) (mid 88.02132 95.13332) (end 85.9 96.012) (stroke (width 0.1) (type default)) (layer "Edge.Cuts"))
 (gr_arc (start 69.929 149.479) (mid 67.80768 148.60032) (end 66.929 146.479) (stroke (width 0.1) (type default)) (layer "Edge.Cuts"))
 (gr_line (start 78.74 93.012) (end 78.74 83.518) (stroke (width 0.1) (type default)) (layer "Edge.Cuts"))
 (gr_line (start 69.929 80.518) (end 75.74 80.518) (stroke (width 0.1) (type default)) (layer "Edge.Cuts"))
 (gr_line (start 100.838 83.518) (end 100.838 146.479) (stroke (width 0.1) (type default)) (layer "Edge.Cuts"))
 (gr_line (start 88.9 83.518) (end 88.9 93.012) (stroke (width 0.1) (type default)) (layer "Edge.Cuts"))
 (gr_line (start 66.929 146.479) (end 66.929 83.518) (stroke (width 0.1) (type default)) (layer "Edge.Cuts"))
 (gr_arc (start 88.9 83.518) (mid 89.77868 81.39668) (end 91.9 80.518) (stroke (width 0.1) (type default)) (layer "Edge.Cuts"))
 (gr_arc (start 97.838 80.518) (mid 99.95932 81.39668) (end 100.838 83.518) (stroke (width 0.1) (type default)) (layer "Edge.Cuts"))
 (gr_line (start 97.838 149.479) (end 69.929 149.479) (stroke (width 0.1) (type default)) (layer "Edge.Cuts"))
 (gr_arc (start 100.838 146.479) (mid 99.95932 148.60032) (end 97.838 149.479) (stroke (width 0.1) (type default)) (layer "Edge.Cuts"))
 (gr_arc (start 75.74 80.518) (mid 77.86132 81.39668) (end 78.74 83.518) (stroke (width 0.1) (type default)) (layer "Edge.Cuts"))
 (gr_arc (start 66.929 83.518) (mid 67.80768 81.39668) (end 69.929 80.518) (stroke (width 0.1) (type default)) (layer "Edge.Cuts"))
 (gr_arc (start 81.74 96.012) (mid 79.61868 95.13332) (end 78.74 93.012) (stroke (width 0.1) (type default)) (layer "Edge.Cuts"))
 (segment (start 70.612 111.76) (end 76.454 111.76) (width 0.25) (layer "F.Cu") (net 3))
 (segment (start 69.342 113.03) (end 70.612 111.76) (width 0.25) (layer "F.Cu") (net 3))
 (segment (start 76.454 111.76) (end 89.027 124.333) (width 0.25) (layer "F.Cu") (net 3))
 (segment (start 89.027 133.477) (end 83.82 138.684) (width 0.25) (layer "F.Cu") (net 3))
 (segment (start 89.027 124.333) (end 89.027 133.477) (width 0.25) (layer "F.Cu") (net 3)))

